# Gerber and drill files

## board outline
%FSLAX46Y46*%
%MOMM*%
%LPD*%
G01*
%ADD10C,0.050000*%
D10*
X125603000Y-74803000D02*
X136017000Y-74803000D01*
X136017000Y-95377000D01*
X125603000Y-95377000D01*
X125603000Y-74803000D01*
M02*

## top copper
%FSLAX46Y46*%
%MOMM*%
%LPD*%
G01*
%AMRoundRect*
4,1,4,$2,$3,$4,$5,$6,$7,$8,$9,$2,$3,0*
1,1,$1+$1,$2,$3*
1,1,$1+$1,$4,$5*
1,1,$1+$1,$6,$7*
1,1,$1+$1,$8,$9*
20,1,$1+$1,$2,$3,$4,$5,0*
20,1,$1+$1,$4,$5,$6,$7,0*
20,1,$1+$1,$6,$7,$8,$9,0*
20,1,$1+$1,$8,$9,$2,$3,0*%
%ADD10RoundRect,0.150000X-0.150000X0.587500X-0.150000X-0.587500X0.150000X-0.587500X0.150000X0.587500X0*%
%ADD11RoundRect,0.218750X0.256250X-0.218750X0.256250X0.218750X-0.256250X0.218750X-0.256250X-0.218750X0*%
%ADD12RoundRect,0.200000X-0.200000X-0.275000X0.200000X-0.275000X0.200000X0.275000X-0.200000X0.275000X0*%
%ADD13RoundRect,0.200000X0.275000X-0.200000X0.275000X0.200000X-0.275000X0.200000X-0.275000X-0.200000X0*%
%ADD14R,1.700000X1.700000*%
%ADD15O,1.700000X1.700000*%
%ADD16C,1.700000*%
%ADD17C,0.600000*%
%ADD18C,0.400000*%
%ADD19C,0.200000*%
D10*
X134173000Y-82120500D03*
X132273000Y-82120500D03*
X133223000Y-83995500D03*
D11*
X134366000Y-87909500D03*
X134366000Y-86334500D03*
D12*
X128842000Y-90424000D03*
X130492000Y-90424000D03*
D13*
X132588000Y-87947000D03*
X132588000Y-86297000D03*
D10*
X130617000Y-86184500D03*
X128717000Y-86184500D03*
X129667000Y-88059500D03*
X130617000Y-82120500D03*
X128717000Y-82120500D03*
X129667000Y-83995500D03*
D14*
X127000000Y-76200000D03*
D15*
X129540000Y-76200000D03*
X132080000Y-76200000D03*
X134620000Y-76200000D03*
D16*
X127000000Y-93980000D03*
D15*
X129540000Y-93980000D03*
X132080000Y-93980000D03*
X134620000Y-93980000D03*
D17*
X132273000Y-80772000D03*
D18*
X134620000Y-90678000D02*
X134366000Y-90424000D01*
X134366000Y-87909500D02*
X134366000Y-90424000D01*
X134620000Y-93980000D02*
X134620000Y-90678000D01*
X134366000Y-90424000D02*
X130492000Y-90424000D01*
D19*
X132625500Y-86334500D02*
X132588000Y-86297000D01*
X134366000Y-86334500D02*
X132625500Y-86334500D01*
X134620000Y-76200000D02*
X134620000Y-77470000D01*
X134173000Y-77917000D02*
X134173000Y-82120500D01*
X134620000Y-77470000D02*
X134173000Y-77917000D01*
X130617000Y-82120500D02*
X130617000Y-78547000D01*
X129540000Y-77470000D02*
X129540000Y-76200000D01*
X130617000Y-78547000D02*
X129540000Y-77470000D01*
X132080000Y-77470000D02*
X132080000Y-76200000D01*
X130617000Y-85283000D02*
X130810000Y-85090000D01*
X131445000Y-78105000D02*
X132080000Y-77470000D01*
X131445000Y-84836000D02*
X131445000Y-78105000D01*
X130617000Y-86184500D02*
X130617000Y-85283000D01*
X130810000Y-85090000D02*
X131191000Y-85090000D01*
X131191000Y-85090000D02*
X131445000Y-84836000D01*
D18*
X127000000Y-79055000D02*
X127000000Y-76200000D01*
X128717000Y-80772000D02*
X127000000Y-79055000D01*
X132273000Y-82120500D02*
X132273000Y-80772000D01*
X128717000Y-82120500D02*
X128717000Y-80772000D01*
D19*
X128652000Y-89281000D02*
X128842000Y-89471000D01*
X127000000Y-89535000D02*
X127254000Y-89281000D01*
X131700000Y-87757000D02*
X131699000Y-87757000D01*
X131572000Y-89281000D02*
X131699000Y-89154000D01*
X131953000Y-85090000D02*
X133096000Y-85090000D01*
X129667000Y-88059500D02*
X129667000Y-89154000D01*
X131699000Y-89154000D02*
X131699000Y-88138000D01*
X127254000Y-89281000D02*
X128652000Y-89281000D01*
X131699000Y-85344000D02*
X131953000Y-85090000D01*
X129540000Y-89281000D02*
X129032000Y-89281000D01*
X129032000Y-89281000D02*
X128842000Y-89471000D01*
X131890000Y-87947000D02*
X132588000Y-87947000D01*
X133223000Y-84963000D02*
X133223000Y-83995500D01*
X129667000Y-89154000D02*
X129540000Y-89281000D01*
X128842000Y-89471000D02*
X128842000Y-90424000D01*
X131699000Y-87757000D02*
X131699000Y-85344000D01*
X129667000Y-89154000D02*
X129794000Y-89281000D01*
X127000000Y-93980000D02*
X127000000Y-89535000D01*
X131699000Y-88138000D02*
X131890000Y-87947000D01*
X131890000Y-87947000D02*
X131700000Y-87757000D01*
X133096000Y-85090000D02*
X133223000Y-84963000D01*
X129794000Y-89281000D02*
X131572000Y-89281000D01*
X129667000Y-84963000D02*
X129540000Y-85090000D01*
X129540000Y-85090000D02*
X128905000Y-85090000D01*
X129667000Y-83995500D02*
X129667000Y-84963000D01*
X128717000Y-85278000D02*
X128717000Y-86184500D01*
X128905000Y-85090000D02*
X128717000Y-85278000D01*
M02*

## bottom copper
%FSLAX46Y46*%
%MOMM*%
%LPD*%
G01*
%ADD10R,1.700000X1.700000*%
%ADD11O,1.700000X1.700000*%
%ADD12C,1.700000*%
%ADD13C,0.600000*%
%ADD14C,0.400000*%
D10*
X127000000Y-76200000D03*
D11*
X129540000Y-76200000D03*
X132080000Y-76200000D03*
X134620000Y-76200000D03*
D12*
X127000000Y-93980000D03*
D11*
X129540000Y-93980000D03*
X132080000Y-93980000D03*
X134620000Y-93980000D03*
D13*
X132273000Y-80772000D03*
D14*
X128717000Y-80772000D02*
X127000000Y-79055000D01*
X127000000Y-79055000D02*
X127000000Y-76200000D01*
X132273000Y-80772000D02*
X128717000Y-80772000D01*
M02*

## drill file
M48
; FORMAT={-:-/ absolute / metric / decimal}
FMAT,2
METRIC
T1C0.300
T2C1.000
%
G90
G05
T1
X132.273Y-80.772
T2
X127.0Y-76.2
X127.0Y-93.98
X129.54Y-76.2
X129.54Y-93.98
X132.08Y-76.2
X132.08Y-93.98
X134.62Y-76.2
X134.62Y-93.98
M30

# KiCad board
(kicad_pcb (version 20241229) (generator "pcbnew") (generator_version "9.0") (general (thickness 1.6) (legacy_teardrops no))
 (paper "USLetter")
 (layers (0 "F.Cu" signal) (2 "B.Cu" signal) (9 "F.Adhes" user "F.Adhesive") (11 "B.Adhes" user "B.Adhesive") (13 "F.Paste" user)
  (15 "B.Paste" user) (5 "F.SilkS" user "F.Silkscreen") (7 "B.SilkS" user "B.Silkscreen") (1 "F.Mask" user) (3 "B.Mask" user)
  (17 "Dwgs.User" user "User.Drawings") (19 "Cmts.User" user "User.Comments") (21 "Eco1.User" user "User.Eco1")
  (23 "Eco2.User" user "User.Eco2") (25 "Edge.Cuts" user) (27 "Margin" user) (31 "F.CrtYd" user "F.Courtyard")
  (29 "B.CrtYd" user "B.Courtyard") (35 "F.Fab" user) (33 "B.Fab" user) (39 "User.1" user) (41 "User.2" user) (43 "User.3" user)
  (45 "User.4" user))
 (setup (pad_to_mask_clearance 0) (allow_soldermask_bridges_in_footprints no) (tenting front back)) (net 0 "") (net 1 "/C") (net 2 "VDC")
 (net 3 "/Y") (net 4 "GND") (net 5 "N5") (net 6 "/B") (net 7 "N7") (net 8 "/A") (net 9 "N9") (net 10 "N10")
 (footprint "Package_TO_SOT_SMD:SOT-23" (layer "F.Cu") (at 133.223 83.058 -90)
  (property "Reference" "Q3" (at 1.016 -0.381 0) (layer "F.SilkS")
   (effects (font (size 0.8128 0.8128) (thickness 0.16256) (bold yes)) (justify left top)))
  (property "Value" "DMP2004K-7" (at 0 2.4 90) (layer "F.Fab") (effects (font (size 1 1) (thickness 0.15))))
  (pad "1" smd roundrect (at -0.9375 -0.95 270) (size 1.475 0.6) (layers "F.Cu" "F.Mask" "F.Paste") (roundrect_rratio 0.25) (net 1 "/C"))
  (pad "2" smd roundrect (at -0.9375 0.95 270) (size 1.475 0.6) (layers "F.Cu" "F.Mask" "F.Paste") (roundrect_rratio 0.25) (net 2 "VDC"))
  (pad "3" smd roundrect (at 0.9375 0 270) (size 1.475 0.6) (layers "F.Cu" "F.Mask" "F.Paste") (roundrect_rratio 0.25) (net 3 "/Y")))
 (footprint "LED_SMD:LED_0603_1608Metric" (layer "F.Cu") (at 134.366 87.122 90)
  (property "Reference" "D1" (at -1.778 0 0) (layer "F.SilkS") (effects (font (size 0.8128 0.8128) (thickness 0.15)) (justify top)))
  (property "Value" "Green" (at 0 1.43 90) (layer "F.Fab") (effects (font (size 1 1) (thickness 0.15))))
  (pad "1" smd roundrect (at -0.7875 0 90) (size 0.875 0.95) (layers "F.Cu" "F.Mask" "F.Paste") (roundrect_rratio 0.25) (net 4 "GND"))
  (pad "2" smd roundrect (at 0.7875 0 90) (size 0.875 0.95) (layers "F.Cu" "F.Mask" "F.Paste") (roundrect_rratio 0.25) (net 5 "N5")))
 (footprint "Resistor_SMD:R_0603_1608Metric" (layer "F.Cu") (at 129.667 90.424)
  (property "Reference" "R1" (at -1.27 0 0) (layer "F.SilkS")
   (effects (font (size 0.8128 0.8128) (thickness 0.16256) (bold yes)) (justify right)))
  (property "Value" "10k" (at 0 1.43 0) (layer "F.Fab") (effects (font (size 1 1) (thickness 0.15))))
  (pad "1" smd roundrect (at -0.825 0) (size 0.8 0.95) (layers "F.Cu" "F.Mask" "F.Paste") (roundrect_rratio 0.25) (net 3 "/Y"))
  (pad "2" smd roundrect (at 0.825 0) (size 0.8 0.95) (layers "F.Cu" "F.Mask" "F.Paste") (roundrect_rratio 0.25) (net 4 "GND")))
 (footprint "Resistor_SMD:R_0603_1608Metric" (layer "F.Cu") (at 132.588 87.122 90)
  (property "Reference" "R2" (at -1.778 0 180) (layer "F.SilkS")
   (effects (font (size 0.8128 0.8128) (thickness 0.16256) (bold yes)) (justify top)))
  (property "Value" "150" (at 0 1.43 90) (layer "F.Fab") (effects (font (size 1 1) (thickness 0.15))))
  (pad "1" smd roundrect (at -0.825 0 90) (size 0.8 0.95) (layers "F.Cu" "F.Mask" "F.Paste") (roundrect_rratio 0.25) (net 3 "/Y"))
  (pad "2" smd roundrect (at 0.825 0 90) (size 0.8 0.95) (layers "F.Cu" "F.Mask" "F.Paste") (roundrect_rratio 0.25) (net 5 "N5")))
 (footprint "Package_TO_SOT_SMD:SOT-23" (layer "F.Cu") (at 129.667 87.122 -90)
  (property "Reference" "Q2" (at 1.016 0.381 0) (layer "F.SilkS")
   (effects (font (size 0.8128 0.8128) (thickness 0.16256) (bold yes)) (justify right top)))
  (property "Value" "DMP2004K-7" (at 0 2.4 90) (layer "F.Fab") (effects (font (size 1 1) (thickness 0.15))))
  (pad "1" smd roundrect (at -0.9375 -0.95 270) (size 1.475 0.6) (layers "F.Cu" "F.Mask" "F.Paste") (roundrect_rratio 0.25) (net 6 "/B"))
  (pad "2" smd roundrect (at -0.9375 0.95 270) (size 1.475 0.6) (layers "F.Cu" "F.Mask" "F.Paste") (roundrect_rratio 0.25) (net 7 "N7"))
  (pad "3" smd roundrect (at 0.9375 0 270) (size 1.475 0.6) (layers "F.Cu" "F.Mask" "F.Paste") (roundrect_rratio 0.25) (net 3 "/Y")))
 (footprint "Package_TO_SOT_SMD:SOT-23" (layer "F.Cu") (at 129.667 83.058 -90)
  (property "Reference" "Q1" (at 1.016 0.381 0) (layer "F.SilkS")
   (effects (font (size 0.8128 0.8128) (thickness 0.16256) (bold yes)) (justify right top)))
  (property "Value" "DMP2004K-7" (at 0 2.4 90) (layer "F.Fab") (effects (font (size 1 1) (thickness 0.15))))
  (pad "1" smd roundrect (at -0.9375 -0.95 270) (size 1.475 0.6) (layers "F.Cu" "F.Mask" "F.Paste") (roundrect_rratio 0.25) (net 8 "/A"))
  (pad "2" smd roundrect (at -0.9375 0.95 270) (size 1.475 0.6) (layers "F.Cu" "F.Mask" "F.Paste") (roundrect_rratio 0.25) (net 2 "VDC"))
  (pad "3" smd roundrect (at 0.9375 0 270) (size 1.475 0.6) (layers "F.Cu" "F.Mask" "F.Paste") (roundrect_rratio 0.25) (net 7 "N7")))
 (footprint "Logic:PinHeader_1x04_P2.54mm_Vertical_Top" (layer "B.Cu") (at 127 76.2 -90)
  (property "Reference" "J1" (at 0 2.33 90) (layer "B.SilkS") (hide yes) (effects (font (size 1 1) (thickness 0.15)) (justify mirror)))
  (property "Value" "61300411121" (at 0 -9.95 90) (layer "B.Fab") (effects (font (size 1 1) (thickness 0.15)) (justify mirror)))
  (pad "1" thru_hole rect (at 0 0 270) (size 1.7 1.7) (drill 1) (layers "*.Cu" "*.Mask") (remove_unused_layers no) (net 2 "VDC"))
  (pad "2" thru_hole oval (at 0 -2.54 270) (size 1.7 1.7) (drill 1) (layers "*.Cu" "*.Mask") (remove_unused_layers no) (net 8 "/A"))
  (pad "3" thru_hole oval (at 0 -5.08 270) (size 1.7 1.7) (drill 1) (layers "*.Cu" "*.Mask") (remove_unused_layers no) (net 6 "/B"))
  (pad "4" thru_hole oval (at 0 -7.62 270) (size 1.7 1.7) (drill 1) (layers "*.Cu" "*.Mask") (remove_unused_layers no) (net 1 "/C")))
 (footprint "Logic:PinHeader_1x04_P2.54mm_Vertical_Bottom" (layer "B.Cu") (at 127 93.98 -90)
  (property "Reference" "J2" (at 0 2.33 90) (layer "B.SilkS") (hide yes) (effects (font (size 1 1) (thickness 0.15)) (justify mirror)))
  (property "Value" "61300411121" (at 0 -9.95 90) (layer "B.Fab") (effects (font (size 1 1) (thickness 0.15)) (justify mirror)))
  (pad "1" thru_hole circle (at 0 0 270) (size 1.7 1.7) (drill 1) (layers "*.Cu" "*.Mask") (remove_unused_layers no) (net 3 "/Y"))
  (pad "2" thru_hole oval (at 0 -2.54 270) (size 1.7 1.7) (drill 1) (layers "*.Cu" "*.Mask") (remove_unused_layers no) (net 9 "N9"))
  (pad "3" thru_hole oval (at 0 -5.08 270) (size 1.7 1.7) (drill 1) (layers "*.Cu" "*.Mask") (remove_unused_layers no) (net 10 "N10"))
  (pad "4" thru_hole oval (at 0 -7.62 270) (size 1.7 1.7) (drill 1) (layers "*.Cu" "*.Mask") (remove_unused_layers no) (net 4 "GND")))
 (gr_rect (start 125.603 74.803) (end 136.017 95.377) (stroke (width 0.05) (type default)) (fill no) (layer "Edge.Cuts"))
 (segment (start 134.62 90.678) (end 134.366 90.424) (width 0.4) (layer "F.Cu") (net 4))
 (segment (start 134.366 87.9095) (end 134.366 90.424) (width 0.4) (layer "F.Cu") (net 4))
 (segment (start 134.62 93.98) (end 134.62 90.678) (width 0.4) (layer "F.Cu") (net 4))
 (segment (start 134.366 90.424) (end 130.492 90.424) (width 0.4) (layer "F.Cu") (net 4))
 (segment (start 132.6255 86.3345) (end 132.588 86.297) (width 0.2) (layer "F.Cu") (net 5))
 (segment (start 134.366 86.3345) (end 132.6255 86.3345) (width 0.2) (layer "F.Cu") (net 5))
 (segment (start 134.62 76.2) (end 134.62 77.47) (width 0.2) (layer "F.Cu") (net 1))
 (segment (start 134.173 77.917) (end 134.173 82.1205) (width 0.2) (layer "F.Cu") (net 1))
 (segment (start 134.62 77.47) (end 134.173 77.917) (width 0.2) (layer "F.Cu") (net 1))
 (segment (start 130.617 82.1205) (end 130.617 78.547) (width 0.2) (layer "F.Cu") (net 8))
 (segment (start 129.54 77.47) (end 129.54 76.2) (width 0.2) (layer "F.Cu") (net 8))
 (segment (start 130.617 78.547) (end 129.54 77.47) (width 0.2) (layer "F.Cu") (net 8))
 (segment (start 132.08 77.47) (end 132.08 76.2) (width 0.2) (layer "F.Cu") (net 6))
 (segment (start 130.617 85.283) (end 130.81 85.09) (width 0.2) (layer "F.Cu") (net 6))
 (segment (start 131.445 78.105) (end 132.08 77.47) (width 0.2) (layer "F.Cu") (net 6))
 (segment (start 131.445 84.836) (end 131.445 78.105) (width 0.2) (layer "F.Cu") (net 6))
 (segment (start 130.617 86.1845) (end 130.617 85.283) (width 0.2) (layer "F.Cu") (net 6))
 (segment (start 130.81 85.09) (end 131.191 85.09) (width 0.2) (layer "F.Cu") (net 6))
 (segment (start 131.191 85.09) (end 131.445 84.836) (width 0.2) (layer "F.Cu") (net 6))
 (segment (start 127 79.055) (end 127 76.2) (width 0.4) (layer "F.Cu") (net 2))
 (segment (start 128.717 80.772) (end 127 79.055) (width 0.4) (layer "F.Cu") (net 2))
 (segment (start 132.273 82.1205) (end 132.273 80.772) (width 0.4) (layer "F.Cu") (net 2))
 (segment (start 128.717 82.1205) (end 128.717 80.772) (width 0.4) (layer "F.Cu") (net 2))
 (via (at 132.273 80.772) (size 0.6) (drill 0.3) (layers "F.Cu" "B.Cu") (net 2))
 (segment (start 128.717 80.772) (end 127 79.055) (width 0.4) (layer "B.Cu") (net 2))
 (segment (start 127 79.055) (end 127 76.2) (width 0.4) (layer "B.Cu") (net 2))
 (segment (start 132.273 80.772) (end 128.717 80.772) (width 0.4) (layer "B.Cu") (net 2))
 (segment (start 128.652 89.281) (end 128.842 89.471) (width 0.2) (layer "F.Cu") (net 3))
 (segment (start 127 89.535) (end 127.254 89.281) (width 0.2) (layer "F.Cu") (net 3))
 (segment (start 131.7 87.757) (end 131.699 87.757) (width 0.2) (layer "F.Cu") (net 3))
 (segment (start 131.572 89.281) (end 131.699 89.154) (width 0.2) (layer "F.Cu") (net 3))
 (segment (start 131.953 85.09) (end 133.096 85.09) (width 0.2) (layer "F.Cu") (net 3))
 (segment (start 129.667 88.0595) (end 129.667 89.154) (width 0.2) (layer "F.Cu") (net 3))
 (segment (start 131.699 89.154) (end 131.699 88.138) (width 0.2) (layer "F.Cu") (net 3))
 (segment (start 127.254 89.281) (end 128.652 89.281) (width 0.2) (layer "F.Cu") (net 3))
 (segment (start 131.699 85.344) (end 131.953 85.09) (width 0.2) (layer "F.Cu") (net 3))
 (segment (start 129.54 89.281) (end 129.032 89.281) (width 0.2) (layer "F.Cu") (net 3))
 (segment (start 129.032 89.281) (end 128.842 89.471) (width 0.2) (layer "F.Cu") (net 3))
 (segment (start 131.89 87.947) (end 132.588 87.947) (width 0.2) (layer "F.Cu") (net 3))
 (segment (start 133.223 84.963) (end 133.223 83.9955) (width 0.2) (layer "F.Cu") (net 3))
 (segment (start 129.667 89.154) (end 129.54 89.281) (width 0.2) (layer "F.Cu") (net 3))
 (segment (start 128.842 89.471) (end 128.842 90.424) (width 0.2) (layer "F.Cu") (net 3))
 (segment (start 131.699 87.757) (end 131.699 85.344) (width 0.2) (layer "F.Cu") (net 3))
 (segment (start 129.667 89.154) (end 129.794 89.281) (width 0.2) (layer "F.Cu") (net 3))
 (segment (start 127 93.98) (end 127 89.535) (width 0.2) (layer "F.Cu") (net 3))
 (segment (start 131.699 88.138) (end 131.89 87.947) (width 0.2) (layer "F.Cu") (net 3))
 (segment (start 131.89 87.947) (end 131.7 87.757) (width 0.2) (layer "F.Cu") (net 3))
 (segment (start 133.096 85.09) (end 133.223 84.963) (width 0.2) (layer "F.Cu") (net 3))
 (segment (start 129.794 89.281) (end 131.572 89.281) (width 0.2) (layer "F.Cu") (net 3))
 (segment (start 129.667 84.963) (end 129.54 85.09) (width 0.2) (layer "F.Cu") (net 7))
 (segment (start 129.54 85.09) (end 128.905 85.09) (width 0.2) (layer "F.Cu") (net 7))
 (segment (start 129.667 83.9955) (end 129.667 84.963) (width 0.2) (layer "F.Cu") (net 7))
 (segment (start 128.717 85.278) (end 128.717 86.1845) (width 0.2) (layer "F.Cu") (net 7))
 (segment (start 128.905 85.09) (end 128.717 85.278) (width 0.2) (layer "F.Cu") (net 7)))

